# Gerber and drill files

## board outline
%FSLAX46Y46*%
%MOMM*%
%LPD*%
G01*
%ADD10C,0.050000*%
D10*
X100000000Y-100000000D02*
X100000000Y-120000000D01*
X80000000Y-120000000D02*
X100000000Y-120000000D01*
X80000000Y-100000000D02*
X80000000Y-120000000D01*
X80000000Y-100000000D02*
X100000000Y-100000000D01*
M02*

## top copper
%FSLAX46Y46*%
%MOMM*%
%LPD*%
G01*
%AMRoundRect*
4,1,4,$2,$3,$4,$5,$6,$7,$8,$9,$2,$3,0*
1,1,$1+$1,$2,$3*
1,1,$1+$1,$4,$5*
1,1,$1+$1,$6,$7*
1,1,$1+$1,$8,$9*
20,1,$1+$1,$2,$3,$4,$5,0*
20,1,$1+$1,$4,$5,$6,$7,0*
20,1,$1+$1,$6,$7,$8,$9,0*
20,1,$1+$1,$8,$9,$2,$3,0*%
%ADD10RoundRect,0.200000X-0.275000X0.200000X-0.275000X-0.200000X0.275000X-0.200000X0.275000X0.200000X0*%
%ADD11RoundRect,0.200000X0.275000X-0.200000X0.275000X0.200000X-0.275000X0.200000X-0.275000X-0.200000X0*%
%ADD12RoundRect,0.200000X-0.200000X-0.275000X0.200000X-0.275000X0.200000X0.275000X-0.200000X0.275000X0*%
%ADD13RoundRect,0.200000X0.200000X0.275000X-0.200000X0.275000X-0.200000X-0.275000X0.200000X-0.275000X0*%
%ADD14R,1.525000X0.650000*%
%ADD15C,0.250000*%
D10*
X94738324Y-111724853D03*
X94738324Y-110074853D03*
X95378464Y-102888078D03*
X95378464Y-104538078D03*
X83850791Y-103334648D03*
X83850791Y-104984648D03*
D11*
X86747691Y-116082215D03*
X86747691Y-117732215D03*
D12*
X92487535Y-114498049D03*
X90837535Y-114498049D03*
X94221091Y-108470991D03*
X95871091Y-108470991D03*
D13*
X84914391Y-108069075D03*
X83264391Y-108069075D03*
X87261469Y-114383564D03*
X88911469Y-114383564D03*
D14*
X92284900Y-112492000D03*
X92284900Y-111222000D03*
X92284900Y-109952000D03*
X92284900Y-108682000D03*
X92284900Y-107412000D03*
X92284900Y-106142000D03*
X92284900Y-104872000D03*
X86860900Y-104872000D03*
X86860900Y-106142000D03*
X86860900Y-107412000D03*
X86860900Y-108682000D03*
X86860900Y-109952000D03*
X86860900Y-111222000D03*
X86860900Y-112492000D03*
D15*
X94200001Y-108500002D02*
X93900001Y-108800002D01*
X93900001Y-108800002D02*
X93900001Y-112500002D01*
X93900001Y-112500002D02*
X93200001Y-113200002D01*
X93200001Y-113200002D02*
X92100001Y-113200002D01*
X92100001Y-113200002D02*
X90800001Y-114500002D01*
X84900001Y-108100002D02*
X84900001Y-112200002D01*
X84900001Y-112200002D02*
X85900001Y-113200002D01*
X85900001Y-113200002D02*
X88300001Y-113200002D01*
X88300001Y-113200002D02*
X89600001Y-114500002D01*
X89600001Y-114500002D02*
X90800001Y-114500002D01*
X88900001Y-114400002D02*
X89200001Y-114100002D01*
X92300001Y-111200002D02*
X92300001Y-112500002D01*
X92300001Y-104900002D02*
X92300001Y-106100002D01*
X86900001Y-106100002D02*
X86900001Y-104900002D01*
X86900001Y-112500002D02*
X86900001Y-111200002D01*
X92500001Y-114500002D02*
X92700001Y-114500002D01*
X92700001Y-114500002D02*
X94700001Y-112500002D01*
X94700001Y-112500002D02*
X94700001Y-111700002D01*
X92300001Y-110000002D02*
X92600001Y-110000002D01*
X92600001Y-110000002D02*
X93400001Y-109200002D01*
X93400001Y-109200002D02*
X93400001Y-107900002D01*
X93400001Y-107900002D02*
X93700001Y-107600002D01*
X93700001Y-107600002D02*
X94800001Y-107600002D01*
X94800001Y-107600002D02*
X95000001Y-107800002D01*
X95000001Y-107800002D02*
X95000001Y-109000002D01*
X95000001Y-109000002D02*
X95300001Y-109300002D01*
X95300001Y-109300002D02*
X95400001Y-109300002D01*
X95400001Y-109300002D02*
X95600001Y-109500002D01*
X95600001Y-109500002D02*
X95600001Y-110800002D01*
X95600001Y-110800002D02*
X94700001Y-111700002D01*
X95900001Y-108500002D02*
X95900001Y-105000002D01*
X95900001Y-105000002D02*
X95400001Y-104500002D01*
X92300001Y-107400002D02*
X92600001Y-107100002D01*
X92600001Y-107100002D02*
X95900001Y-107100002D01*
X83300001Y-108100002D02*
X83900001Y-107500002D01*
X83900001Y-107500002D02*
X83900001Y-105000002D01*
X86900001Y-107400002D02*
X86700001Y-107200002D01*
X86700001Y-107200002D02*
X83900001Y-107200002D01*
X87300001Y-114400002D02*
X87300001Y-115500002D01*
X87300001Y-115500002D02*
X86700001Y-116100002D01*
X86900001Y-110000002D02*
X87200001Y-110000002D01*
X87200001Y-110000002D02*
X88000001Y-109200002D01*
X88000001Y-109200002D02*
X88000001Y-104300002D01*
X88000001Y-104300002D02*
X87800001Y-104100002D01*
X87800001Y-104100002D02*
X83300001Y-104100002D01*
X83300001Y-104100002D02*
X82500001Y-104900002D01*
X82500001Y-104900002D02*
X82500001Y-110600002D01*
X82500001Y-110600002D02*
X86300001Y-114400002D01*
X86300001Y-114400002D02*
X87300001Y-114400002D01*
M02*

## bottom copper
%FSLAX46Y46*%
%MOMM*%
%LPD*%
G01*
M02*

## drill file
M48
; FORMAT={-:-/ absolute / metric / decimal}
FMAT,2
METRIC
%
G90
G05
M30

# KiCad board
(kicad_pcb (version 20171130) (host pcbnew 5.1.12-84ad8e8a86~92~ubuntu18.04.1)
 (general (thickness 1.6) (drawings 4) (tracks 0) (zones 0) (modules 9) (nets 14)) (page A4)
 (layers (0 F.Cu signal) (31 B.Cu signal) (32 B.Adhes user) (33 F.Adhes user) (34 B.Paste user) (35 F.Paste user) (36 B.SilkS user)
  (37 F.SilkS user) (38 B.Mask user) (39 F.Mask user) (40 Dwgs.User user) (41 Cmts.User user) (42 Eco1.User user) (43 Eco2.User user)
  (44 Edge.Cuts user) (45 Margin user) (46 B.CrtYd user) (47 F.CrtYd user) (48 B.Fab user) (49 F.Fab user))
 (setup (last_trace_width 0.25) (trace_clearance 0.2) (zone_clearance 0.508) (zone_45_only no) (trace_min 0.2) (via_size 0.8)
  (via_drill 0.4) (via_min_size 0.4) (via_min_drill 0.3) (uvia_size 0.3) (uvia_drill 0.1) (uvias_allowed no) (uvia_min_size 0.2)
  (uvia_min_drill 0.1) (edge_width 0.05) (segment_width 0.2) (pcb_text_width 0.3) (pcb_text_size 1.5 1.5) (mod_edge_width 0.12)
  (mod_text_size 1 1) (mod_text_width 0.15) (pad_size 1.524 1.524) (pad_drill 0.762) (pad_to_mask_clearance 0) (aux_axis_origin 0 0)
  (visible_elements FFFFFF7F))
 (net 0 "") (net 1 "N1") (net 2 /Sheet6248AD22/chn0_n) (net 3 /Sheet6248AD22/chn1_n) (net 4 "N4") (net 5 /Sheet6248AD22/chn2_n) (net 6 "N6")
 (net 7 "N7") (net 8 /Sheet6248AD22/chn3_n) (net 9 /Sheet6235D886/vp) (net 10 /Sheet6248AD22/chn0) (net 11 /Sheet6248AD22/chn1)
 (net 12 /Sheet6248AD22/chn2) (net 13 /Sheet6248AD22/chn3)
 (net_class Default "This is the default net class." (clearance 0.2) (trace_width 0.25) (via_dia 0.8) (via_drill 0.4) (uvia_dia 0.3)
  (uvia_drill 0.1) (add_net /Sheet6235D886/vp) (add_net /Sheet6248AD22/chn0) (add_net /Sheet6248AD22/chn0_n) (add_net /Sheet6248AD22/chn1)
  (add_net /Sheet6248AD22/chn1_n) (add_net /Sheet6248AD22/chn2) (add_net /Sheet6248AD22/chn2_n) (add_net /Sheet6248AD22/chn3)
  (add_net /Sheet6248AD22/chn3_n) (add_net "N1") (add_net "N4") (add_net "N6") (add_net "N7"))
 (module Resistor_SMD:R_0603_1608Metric (layer F.Cu) (at 94.738324 110.899853 270.000000)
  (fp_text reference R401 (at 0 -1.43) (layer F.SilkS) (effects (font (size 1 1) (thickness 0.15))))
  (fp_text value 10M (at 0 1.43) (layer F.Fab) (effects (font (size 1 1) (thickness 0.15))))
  (pad 2 smd roundrect (at 0.825 0 270.000000) (size 0.8 0.95) (layers F.Cu F.Mask F.Paste) (roundrect_rratio 0.25) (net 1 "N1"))
  (pad 1 smd roundrect (at -0.825 0 270.000000) (size 0.8 0.95) (layers F.Cu F.Mask F.Paste) (roundrect_rratio 0.25)
   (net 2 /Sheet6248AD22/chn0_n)))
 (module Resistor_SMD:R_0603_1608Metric (layer F.Cu) (at 95.378464 103.713078 270.000000)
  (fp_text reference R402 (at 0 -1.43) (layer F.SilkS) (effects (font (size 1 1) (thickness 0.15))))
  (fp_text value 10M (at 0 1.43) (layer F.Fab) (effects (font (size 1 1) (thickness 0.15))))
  (pad 1 smd roundrect (at -0.825 0 270.000000) (size 0.8 0.95) (layers F.Cu F.Mask F.Paste) (roundrect_rratio 0.25)
   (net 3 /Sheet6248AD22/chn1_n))
  (pad 2 smd roundrect (at 0.825 0 270.000000) (size 0.8 0.95) (layers F.Cu F.Mask F.Paste) (roundrect_rratio 0.25) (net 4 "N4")))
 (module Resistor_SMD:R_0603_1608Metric (layer F.Cu) (at 83.850791 104.159648 270.000000)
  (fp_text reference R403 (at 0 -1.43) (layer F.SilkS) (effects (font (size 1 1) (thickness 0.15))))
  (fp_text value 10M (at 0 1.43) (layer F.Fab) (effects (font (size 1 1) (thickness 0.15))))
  (pad 1 smd roundrect (at -0.825 0 270.000000) (size 0.8 0.95) (layers F.Cu F.Mask F.Paste) (roundrect_rratio 0.25)
   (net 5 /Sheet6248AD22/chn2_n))
  (pad 2 smd roundrect (at 0.825 0 270.000000) (size 0.8 0.95) (layers F.Cu F.Mask F.Paste) (roundrect_rratio 0.25) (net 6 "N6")))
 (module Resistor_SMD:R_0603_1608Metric (layer F.Cu) (at 86.747691 116.907215 90.000000)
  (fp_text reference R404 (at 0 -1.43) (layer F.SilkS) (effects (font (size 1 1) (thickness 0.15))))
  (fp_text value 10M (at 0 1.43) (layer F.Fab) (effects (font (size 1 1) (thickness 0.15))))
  (pad 2 smd roundrect (at 0.825 0 90.000000) (size 0.8 0.95) (layers F.Cu F.Mask F.Paste) (roundrect_rratio 0.25) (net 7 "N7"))
  (pad 1 smd roundrect (at -0.825 0 90.000000) (size 0.8 0.95) (layers F.Cu F.Mask F.Paste) (roundrect_rratio 0.25)
   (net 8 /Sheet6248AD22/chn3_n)))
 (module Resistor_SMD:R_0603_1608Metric (layer F.Cu) (at 91.662535 114.498049)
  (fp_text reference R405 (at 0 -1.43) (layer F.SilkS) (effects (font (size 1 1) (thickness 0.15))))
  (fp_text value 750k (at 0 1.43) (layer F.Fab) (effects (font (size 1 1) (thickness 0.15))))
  (pad 2 smd roundrect (at 0.825 0) (size 0.8 0.95) (layers F.Cu F.Mask F.Paste) (roundrect_rratio 0.25) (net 1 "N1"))
  (pad 1 smd roundrect (at -0.825 0) (size 0.8 0.95) (layers F.Cu F.Mask F.Paste) (roundrect_rratio 0.25) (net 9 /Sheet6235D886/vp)))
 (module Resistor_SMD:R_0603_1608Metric (layer F.Cu) (at 95.046091 108.470991)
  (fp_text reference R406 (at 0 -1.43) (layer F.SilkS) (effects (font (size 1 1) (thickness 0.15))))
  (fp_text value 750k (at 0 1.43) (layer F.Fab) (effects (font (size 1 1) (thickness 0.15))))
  (pad 1 smd roundrect (at -0.825 0) (size 0.8 0.95) (layers F.Cu F.Mask F.Paste) (roundrect_rratio 0.25) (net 9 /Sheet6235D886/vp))
  (pad 2 smd roundrect (at 0.825 0) (size 0.8 0.95) (layers F.Cu F.Mask F.Paste) (roundrect_rratio 0.25) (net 4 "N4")))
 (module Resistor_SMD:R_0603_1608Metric (layer F.Cu) (at 84.089391 108.069075 180.000000)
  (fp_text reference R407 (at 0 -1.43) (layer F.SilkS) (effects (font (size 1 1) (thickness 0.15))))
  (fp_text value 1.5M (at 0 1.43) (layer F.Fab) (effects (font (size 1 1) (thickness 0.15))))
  (pad 1 smd roundrect (at -0.825 0 180.000000) (size 0.8 0.95) (layers F.Cu F.Mask F.Paste) (roundrect_rratio 0.25)
   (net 9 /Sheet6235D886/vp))
  (pad 2 smd roundrect (at 0.825 0 180.000000) (size 0.8 0.95) (layers F.Cu F.Mask F.Paste) (roundrect_rratio 0.25) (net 6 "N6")))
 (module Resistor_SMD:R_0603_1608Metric (layer F.Cu) (at 88.086469 114.383564 180.000000)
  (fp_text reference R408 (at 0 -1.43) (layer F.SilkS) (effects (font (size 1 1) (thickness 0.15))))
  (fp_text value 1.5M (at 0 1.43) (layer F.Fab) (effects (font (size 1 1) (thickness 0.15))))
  (pad 2 smd roundrect (at 0.825 0 180.000000) (size 0.8 0.95) (layers F.Cu F.Mask F.Paste) (roundrect_rratio 0.25) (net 7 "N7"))
  (pad 1 smd roundrect (at -0.825 0 180.000000) (size 0.8 0.95) (layers F.Cu F.Mask F.Paste) (roundrect_rratio 0.25)
   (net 9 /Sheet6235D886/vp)))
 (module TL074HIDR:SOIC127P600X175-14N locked (layer F.Cu) (at 89.572900 108.682000 180.000000)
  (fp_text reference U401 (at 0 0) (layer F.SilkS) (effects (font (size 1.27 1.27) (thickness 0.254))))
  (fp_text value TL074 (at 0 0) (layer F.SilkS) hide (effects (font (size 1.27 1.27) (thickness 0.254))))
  (pad 1 smd rect (at -2.712 -3.81 270.000000) (size 0.65 1.525) (layers F.Cu F.Mask F.Paste) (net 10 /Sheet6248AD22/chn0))
  (pad 2 smd rect (at -2.712 -2.54 270.000000) (size 0.65 1.525) (layers F.Cu F.Mask F.Paste) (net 10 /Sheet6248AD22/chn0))
  (pad 3 smd rect (at -2.712 -1.27 270.000000) (size 0.65 1.525) (layers F.Cu F.Mask F.Paste) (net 1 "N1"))
  (pad 4 smd rect (at -2.712 0 270.000000) (size 0.65 1.525) (layers F.Cu F.Mask F.Paste))
  (pad 5 smd rect (at -2.712 1.27 270.000000) (size 0.65 1.525) (layers F.Cu F.Mask F.Paste) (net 4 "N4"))
  (pad 6 smd rect (at -2.712 2.54 270.000000) (size 0.65 1.525) (layers F.Cu F.Mask F.Paste) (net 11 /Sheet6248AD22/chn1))
  (pad 7 smd rect (at -2.712 3.81 270.000000) (size 0.65 1.525) (layers F.Cu F.Mask F.Paste) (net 11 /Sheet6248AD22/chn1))
  (pad 8 smd rect (at 2.712 3.81 270.000000) (size 0.65 1.525) (layers F.Cu F.Mask F.Paste) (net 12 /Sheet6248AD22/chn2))
  (pad 9 smd rect (at 2.712 2.54 270.000000) (size 0.65 1.525) (layers F.Cu F.Mask F.Paste) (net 12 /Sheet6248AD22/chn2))
  (pad 10 smd rect (at 2.712 1.27 270.000000) (size 0.65 1.525) (layers F.Cu F.Mask F.Paste) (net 6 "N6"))
  (pad 11 smd rect (at 2.712 0 270.000000) (size 0.65 1.525) (layers F.Cu F.Mask F.Paste))
  (pad 12 smd rect (at 2.712 -1.27 270.000000) (size 0.65 1.525) (layers F.Cu F.Mask F.Paste) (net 7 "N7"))
  (pad 13 smd rect (at 2.712 -2.54 270.000000) (size 0.65 1.525) (layers F.Cu F.Mask F.Paste) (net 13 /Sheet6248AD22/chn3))
  (pad 14 smd rect (at 2.712 -3.81 270.000000) (size 0.65 1.525) (layers F.Cu F.Mask F.Paste) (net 13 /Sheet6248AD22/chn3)))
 (gr_line (start 100 100) (end 100 120) (layer Edge.Cuts) (width 0.05))
 (gr_line (start 80 120) (end 100 120) (layer Edge.Cuts) (width 0.05))
 (gr_line (start 80 100) (end 80 120) (layer Edge.Cuts) (width 0.05))
 (gr_line (start 80 100) (end 100 100) (layer Edge.Cuts) (width 0.05))
 (segment (start 94.200001 108.500002) (end 93.900001 108.800002) (width 0.250000) (layer F.Cu) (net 9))
 (segment (start 93.900001 108.800002) (end 93.900001 112.500002) (width 0.250000) (layer F.Cu) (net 9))
 (segment (start 93.900001 112.500002) (end 93.200001 113.200002) (width 0.250000) (layer F.Cu) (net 9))
 (segment (start 93.200001 113.200002) (end 92.100001 113.200002) (width 0.250000) (layer F.Cu) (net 9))
 (segment (start 92.100001 113.200002) (end 90.800001 114.500002) (width 0.250000) (layer F.Cu) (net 9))
 (segment (start 84.900001 108.100002) (end 84.900001 112.200002) (width 0.250000) (layer F.Cu) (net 9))
 (segment (start 84.900001 112.200002) (end 85.900001 113.200002) (width 0.250000) (layer F.Cu) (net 9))
 (segment (start 85.900001 113.200002) (end 88.300001 113.200002) (width 0.250000) (layer F.Cu) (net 9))
 (segment (start 88.300001 113.200002) (end 89.600001 114.500002) (width 0.250000) (layer F.Cu) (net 9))
 (segment (start 89.600001 114.500002) (end 90.800001 114.500002) (width 0.250000) (layer F.Cu) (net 9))
 (segment (start 88.900001 114.400002) (end 89.200001 114.100002) (width 0.250000) (layer F.Cu) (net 9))
 (segment (start 92.300001 111.200002) (end 92.300001 112.500002) (width 0.250000) (layer F.Cu) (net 10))
 (segment (start 92.300001 104.900002) (end 92.300001 106.100002) (width 0.250000) (layer F.Cu) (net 11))
 (segment (start 86.900001 106.100002) (end 86.900001 104.900002) (width 0.250000) (layer F.Cu) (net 12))
 (segment (start 86.900001 112.500002) (end 86.900001 111.200002) (width 0.250000) (layer F.Cu) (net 13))
 (segment (start 92.500001 114.500002) (end 92.700001 114.500002) (width 0.250000) (layer F.Cu) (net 1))
 (segment (start 92.700001 114.500002) (end 94.700001 112.500002) (width 0.250000) (layer F.Cu) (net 1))
 (segment (start 94.700001 112.500002) (end 94.700001 111.700002) (width 0.250000) (layer F.Cu) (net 1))
 (segment (start 92.300001 110.000002) (end 92.600001 110.000002) (width 0.250000) (layer F.Cu) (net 1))
 (segment (start 92.600001 110.000002) (end 93.400001 109.200002) (width 0.250000) (layer F.Cu) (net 1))
 (segment (start 93.400001 109.200002) (end 93.400001 107.900002) (width 0.250000) (layer F.Cu) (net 1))
 (segment (start 93.400001 107.900002) (end 93.700001 107.600002) (width 0.250000) (layer F.Cu) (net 1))
 (segment (start 93.700001 107.600002) (end 94.800001 107.600002) (width 0.250000) (layer F.Cu) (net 1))
 (segment (start 94.800001 107.600002) (end 95.000001 107.800002) (width 0.250000) (layer F.Cu) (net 1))
 (segment (start 95.000001 107.800002) (end 95.000001 109.000002) (width 0.250000) (layer F.Cu) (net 1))
 (segment (start 95.000001 109.000002) (end 95.300001 109.300002) (width 0.250000) (layer F.Cu) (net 1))
 (segment (start 95.300001 109.300002) (end 95.400001 109.300002) (width 0.250000) (layer F.Cu) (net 1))
 (segment (start 95.400001 109.300002) (end 95.600001 109.500002) (width 0.250000) (layer F.Cu) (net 1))
 (segment (start 95.600001 109.500002) (end 95.600001 110.800002) (width 0.250000) (layer F.Cu) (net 1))
 (segment (start 95.600001 110.800002) (end 94.700001 111.700002) (width 0.250000) (layer F.Cu) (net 1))
 (segment (start 95.900001 108.500002) (end 95.900001 105.000002) (width 0.250000) (layer F.Cu) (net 4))
 (segment (start 95.900001 105.000002) (end 95.400001 104.500002) (width 0.250000) (layer F.Cu) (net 4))
 (segment (start 92.300001 107.400002) (end 92.600001 107.100002) (width 0.250000) (layer F.Cu) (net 4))
 (segment (start 92.600001 107.100002) (end 95.900001 107.100002) (width 0.250000) (layer F.Cu) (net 4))
 (segment (start 83.300001 108.100002) (end 83.900001 107.500002) (width 0.250000) (layer F.Cu) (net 6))
 (segment (start 83.900001 107.500002) (end 83.900001 105.000002) (width 0.250000) (layer F.Cu) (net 6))
 (segment (start 86.900001 107.400002) (end 86.700001 107.200002) (width 0.250000) (layer F.Cu) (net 6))
 (segment (start 86.700001 107.200002) (end 83.900001 107.200002) (width 0.250000) (layer F.Cu) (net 6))
 (segment (start 87.300001 114.400002) (end 87.300001 115.500002) (width 0.250000) (layer F.Cu) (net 7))
 (segment (start 87.300001 115.500002) (end 86.700001 116.100002) (width 0.250000) (layer F.Cu) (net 7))
 (segment (start 86.900001 110.000002) (end 87.200001 110.000002) (width 0.250000) (layer F.Cu) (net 7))
 (segment (start 87.200001 110.000002) (end 88.000001 109.200002) (width 0.250000) (layer F.Cu) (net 7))
 (segment (start 88.000001 109.200002) (end 88.000001 104.300002) (width 0.250000) (layer F.Cu) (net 7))
 (segment (start 88.000001 104.300002) (end 87.800001 104.100002) (width 0.250000) (layer F.Cu) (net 7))
 (segment (start 87.800001 104.100002) (end 83.300001 104.100002) (width 0.250000) (layer F.Cu) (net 7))
 (segment (start 83.300001 104.100002) (end 82.500001 104.900002) (width 0.250000) (layer F.Cu) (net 7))
 (segment (start 82.500001 104.900002) (end 82.500001 110.600002) (width 0.250000) (layer F.Cu) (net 7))
 (segment (start 82.500001 110.600002) (end 86.300001 114.400002) (width 0.250000) (layer F.Cu) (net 7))
 (segment (start 86.300001 114.400002) (end 87.300001 114.400002) (width 0.250000) (layer F.Cu) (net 7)))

